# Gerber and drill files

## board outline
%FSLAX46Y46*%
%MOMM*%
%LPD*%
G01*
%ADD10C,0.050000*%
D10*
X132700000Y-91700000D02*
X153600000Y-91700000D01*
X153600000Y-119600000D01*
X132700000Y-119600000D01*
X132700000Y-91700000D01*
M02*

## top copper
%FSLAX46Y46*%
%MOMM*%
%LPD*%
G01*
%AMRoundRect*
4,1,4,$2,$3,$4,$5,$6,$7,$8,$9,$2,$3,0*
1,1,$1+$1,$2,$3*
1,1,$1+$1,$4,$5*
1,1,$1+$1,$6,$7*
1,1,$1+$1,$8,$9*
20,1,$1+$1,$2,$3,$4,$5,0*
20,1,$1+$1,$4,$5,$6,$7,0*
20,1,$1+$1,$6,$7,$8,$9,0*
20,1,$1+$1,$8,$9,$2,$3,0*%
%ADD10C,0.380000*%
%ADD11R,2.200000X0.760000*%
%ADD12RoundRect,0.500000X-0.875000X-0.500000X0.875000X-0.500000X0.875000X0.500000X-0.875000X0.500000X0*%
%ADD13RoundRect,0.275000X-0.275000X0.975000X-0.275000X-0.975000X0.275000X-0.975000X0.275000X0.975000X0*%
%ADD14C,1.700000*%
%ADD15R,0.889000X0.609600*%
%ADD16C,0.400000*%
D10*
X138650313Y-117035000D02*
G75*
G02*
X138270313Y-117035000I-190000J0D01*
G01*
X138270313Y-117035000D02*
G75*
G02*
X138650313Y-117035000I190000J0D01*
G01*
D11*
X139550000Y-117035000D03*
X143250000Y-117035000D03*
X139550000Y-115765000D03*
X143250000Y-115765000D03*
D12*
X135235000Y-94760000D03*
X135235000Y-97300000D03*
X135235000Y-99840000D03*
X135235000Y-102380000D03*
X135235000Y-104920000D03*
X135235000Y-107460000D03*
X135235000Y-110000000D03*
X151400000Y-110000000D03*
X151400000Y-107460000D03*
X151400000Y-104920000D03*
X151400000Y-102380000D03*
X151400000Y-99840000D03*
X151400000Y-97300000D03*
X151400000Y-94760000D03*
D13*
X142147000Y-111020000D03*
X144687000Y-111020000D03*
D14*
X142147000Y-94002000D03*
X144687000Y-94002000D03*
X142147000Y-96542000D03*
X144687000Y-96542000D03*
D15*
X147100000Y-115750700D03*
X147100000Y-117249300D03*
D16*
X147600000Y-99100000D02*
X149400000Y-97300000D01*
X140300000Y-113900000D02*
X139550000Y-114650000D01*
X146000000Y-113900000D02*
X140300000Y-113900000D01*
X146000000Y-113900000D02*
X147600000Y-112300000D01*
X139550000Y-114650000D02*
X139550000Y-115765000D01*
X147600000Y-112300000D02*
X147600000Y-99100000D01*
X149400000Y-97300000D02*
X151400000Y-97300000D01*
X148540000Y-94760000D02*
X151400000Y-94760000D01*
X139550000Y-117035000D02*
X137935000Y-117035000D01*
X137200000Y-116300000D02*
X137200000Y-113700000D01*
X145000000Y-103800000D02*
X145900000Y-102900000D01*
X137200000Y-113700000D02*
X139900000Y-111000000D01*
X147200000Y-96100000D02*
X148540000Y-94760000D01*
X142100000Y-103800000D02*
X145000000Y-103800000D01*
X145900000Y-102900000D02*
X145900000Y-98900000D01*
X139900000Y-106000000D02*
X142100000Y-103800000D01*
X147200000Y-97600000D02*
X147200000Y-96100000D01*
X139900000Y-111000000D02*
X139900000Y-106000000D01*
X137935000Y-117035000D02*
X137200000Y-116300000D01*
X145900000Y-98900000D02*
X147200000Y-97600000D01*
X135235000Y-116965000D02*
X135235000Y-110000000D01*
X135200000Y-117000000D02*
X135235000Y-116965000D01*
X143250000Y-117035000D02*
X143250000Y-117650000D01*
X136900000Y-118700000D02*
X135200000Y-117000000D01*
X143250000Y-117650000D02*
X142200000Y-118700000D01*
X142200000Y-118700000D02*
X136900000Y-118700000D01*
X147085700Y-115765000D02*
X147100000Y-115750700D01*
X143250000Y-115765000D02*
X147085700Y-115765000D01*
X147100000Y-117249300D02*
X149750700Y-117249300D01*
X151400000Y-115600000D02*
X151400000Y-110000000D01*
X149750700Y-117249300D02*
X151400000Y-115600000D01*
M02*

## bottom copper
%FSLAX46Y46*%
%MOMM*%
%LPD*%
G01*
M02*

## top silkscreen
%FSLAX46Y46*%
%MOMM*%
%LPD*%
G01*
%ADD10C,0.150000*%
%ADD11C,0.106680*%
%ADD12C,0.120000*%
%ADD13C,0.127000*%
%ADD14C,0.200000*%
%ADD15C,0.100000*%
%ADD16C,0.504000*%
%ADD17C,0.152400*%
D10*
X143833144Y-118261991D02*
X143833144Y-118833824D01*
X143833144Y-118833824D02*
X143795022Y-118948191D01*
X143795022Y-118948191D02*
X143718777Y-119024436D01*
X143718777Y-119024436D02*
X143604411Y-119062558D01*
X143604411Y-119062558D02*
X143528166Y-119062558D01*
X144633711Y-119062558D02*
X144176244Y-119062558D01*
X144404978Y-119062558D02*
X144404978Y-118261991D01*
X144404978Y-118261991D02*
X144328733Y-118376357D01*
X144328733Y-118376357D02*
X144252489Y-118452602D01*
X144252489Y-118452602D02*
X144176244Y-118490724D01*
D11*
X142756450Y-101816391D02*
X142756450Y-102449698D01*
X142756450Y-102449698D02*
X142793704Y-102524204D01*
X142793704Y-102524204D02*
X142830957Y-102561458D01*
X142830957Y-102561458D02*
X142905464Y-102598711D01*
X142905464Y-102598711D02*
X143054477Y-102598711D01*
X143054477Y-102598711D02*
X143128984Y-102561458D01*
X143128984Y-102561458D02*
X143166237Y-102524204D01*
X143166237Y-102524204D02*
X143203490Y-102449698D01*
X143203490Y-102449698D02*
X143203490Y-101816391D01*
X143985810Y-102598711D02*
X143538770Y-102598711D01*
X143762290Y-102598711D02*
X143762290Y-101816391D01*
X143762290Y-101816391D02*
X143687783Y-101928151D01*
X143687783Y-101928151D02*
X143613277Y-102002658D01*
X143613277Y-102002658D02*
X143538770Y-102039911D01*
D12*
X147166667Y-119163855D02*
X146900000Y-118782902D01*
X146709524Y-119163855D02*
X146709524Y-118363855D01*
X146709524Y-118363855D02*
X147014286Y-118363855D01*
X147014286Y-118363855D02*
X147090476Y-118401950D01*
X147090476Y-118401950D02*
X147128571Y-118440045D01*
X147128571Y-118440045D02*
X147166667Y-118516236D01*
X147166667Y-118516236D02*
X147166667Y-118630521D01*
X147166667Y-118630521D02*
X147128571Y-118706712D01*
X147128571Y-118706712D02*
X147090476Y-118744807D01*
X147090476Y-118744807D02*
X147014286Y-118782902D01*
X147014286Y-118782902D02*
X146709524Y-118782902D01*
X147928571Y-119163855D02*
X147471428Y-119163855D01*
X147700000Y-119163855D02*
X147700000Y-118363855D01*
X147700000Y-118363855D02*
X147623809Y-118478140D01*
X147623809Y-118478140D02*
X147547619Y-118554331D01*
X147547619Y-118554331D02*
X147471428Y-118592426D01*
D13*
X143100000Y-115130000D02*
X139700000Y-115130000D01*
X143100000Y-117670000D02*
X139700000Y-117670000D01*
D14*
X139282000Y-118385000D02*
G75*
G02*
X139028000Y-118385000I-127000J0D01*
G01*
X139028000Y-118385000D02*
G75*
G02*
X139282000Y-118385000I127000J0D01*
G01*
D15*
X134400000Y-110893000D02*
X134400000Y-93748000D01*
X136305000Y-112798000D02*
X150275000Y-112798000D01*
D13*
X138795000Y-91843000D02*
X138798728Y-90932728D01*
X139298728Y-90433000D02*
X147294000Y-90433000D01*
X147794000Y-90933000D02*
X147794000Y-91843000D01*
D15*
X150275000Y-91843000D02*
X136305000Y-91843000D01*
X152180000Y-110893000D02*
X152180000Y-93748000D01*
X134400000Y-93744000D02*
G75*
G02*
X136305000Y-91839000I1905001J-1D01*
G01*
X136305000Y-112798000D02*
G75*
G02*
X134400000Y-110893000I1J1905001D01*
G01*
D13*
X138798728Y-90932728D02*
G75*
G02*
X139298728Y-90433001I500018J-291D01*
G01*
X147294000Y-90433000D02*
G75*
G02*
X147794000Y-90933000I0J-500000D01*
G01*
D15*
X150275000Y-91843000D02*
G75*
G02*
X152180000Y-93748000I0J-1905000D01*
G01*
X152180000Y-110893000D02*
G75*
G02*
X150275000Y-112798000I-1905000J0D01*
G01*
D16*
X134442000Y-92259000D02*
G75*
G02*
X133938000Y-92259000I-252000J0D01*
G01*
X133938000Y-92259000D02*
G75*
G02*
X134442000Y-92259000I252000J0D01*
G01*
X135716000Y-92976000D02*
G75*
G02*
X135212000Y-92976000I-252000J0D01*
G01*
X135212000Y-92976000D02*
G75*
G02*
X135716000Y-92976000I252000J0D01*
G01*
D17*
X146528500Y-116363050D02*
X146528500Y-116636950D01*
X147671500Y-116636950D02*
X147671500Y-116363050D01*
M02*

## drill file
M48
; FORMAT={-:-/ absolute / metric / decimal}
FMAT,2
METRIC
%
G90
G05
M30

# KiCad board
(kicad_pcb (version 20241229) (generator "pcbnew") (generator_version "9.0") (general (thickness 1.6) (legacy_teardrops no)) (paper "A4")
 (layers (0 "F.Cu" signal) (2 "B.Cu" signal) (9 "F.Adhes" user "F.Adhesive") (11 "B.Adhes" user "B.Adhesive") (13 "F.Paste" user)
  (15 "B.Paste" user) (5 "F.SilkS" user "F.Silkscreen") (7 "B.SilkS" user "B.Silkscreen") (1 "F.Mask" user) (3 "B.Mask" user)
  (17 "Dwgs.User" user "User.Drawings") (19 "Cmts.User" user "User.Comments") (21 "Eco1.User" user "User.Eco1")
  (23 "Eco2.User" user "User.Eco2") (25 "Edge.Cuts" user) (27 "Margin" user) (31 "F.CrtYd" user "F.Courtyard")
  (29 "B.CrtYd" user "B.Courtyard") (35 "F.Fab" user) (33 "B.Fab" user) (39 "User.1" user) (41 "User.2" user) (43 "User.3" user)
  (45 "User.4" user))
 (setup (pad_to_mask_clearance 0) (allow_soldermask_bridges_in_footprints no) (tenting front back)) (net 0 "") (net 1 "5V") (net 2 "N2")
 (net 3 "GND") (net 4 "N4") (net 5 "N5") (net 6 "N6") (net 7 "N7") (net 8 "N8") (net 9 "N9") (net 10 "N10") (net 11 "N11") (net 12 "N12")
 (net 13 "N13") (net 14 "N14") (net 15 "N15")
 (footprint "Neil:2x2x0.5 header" (layer "F.Cu") (at 141.4 116.4 90)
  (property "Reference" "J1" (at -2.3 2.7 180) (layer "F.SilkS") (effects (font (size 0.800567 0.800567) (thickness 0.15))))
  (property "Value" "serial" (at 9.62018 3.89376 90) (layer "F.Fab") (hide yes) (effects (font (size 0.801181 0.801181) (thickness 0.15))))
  (fp_line (start 1.27 1.7) (end 1.27 -1.7) (stroke (width 0.127) (type solid)) (layer "F.SilkS"))
  (fp_line (start -1.27 1.7) (end -1.27 -1.7) (stroke (width 0.127) (type solid)) (layer "F.SilkS"))
  (fp_circle (center -1.985 -2.245) (end -1.858 -2.245) (stroke (width 0.2) (type solid)) (fill no) (layer "F.SilkS"))
  (pad "1" smd rect (at -0.635 -1.85 90) (size 0.76 2.2) (layers "F.Cu" "F.Mask" "F.Paste") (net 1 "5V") (solder_mask_margin 0.102))
  (pad "2" smd rect (at -0.635 1.85 90) (size 0.76 2.2) (layers "F.Cu" "F.Mask" "F.Paste") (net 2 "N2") (solder_mask_margin 0.102))
  (pad "3" smd rect (at 0.635 -1.85 90) (size 0.76 2.2) (layers "F.Cu" "F.Mask" "F.Paste") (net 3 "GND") (solder_mask_margin 0.102))
  (pad "4" smd rect (at 0.635 1.85 90) (size 0.76 2.2) (layers "F.Cu" "F.Mask" "F.Paste") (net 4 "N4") (solder_mask_margin 0.102)))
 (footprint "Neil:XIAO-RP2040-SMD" (layer "F.Cu") (at 143.235 102.38)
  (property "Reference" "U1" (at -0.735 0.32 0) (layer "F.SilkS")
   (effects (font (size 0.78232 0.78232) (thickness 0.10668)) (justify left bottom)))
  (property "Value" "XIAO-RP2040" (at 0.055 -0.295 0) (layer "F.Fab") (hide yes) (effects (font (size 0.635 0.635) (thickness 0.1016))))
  (fp_line (start -8.835 8.513) (end -8.835 -8.632) (stroke (width 0.1) (type solid)) (layer "F.SilkS"))
  (fp_line (start -6.93 10.418) (end 7.04 10.418) (stroke (width 0.1) (type solid)) (layer "F.SilkS"))
  (fp_line (start -4.44 -10.537) (end -4.436272 -11.447272) (stroke (width 0.127) (type solid)) (layer "F.SilkS"))
  (fp_line (start -3.936272 -11.947) (end 4.059 -11.947) (stroke (width 0.127) (type solid)) (layer "F.SilkS"))
  (fp_line (start 4.559 -11.447) (end 4.559 -10.537) (stroke (width 0.127) (type solid)) (layer "F.SilkS"))
  (fp_line (start 7.04 -10.537) (end -6.93 -10.537) (stroke (width 0.1) (type solid)) (layer "F.SilkS"))
  (fp_line (start 8.945 8.513) (end 8.945 -8.632) (stroke (width 0.1) (type solid)) (layer "F.SilkS"))
  (fp_arc (start -8.835 -8.636) (mid -8.277038 -9.983038) (end -6.93 -10.541) (stroke (width 0.1) (type solid)) (layer "F.SilkS"))
  (fp_arc (start -6.93 10.418) (mid -8.277038 9.860038) (end -8.835 8.513) (stroke (width 0.1) (type solid)) (layer "F.SilkS"))
  (fp_arc (start -4.436272 -11.447272) (mid -4.289724 -11.800644) (end -3.936272 -11.947) (stroke (width 0.127) (type default))
   (layer "F.SilkS"))
  (fp_arc (start 4.059 -11.947) (mid 4.412553 -11.800553) (end 4.559 -11.447) (stroke (width 0.127) (type default)) (layer "F.SilkS"))
  (fp_arc (start 7.04 -10.537) (mid 8.387038 -9.979038) (end 8.945 -8.632) (stroke (width 0.1) (type solid)) (layer "F.SilkS"))
  (fp_arc (start 8.945 8.513) (mid 8.387038 9.860038) (end 7.04 10.418) (stroke (width 0.1) (type solid)) (layer "F.SilkS"))
  (fp_circle (center -9.045 -10.121) (end -9.045 -10.375) (stroke (width 0.5) (type solid)) (fill yes) (layer "F.SilkS"))
  (fp_circle (center -7.771 -9.404) (end -7.771 -9.658) (stroke (width 0.5) (type solid)) (fill yes) (layer "F.SilkS"))
  (pad "1" smd roundrect (at -8 -7.62) (size 2.75 2) (layers "F.Cu" "F.Mask" "F.Paste") (roundrect_rratio 0.25) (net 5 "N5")
   (solder_mask_margin 0.0508) (thermal_bridge_angle 45))
  (pad "2" smd roundrect (at -8 -5.08) (size 2.75 2) (layers "F.Cu" "F.Mask" "F.Paste") (roundrect_rratio 0.25) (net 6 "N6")
   (solder_mask_margin 0.0508) (thermal_bridge_angle 45))
  (pad "3" smd roundrect (at -8 -2.54) (size 2.75 2) (layers "F.Cu" "F.Mask" "F.Paste") (roundrect_rratio 0.25) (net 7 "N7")
   (solder_mask_margin 0.0508) (thermal_bridge_angle 45))
  (pad "4" smd roundrect (at -8 0) (size 2.75 2) (layers "F.Cu" "F.Mask" "F.Paste") (roundrect_rratio 0.25) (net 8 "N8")
   (solder_mask_margin 0.0508) (thermal_bridge_angle 45))
  (pad "5" smd roundrect (at -8 2.54) (size 2.75 2) (layers "F.Cu" "F.Mask" "F.Paste") (roundrect_rratio 0.25) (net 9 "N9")
   (solder_mask_margin 0.0508) (thermal_bridge_angle 45))
  (pad "6" smd roundrect (at -8 5.08) (size 2.75 2) (layers "F.Cu" "F.Mask" "F.Paste") (roundrect_rratio 0.25) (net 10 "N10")
   (solder_mask_margin 0.0508) (thermal_bridge_angle 45))
  (pad "7" smd roundrect (at -8 7.62) (size 2.75 2) (layers "F.Cu" "F.Mask" "F.Paste") (roundrect_rratio 0.25) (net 2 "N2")
   (solder_mask_margin 0.0508) (thermal_bridge_angle 45))
  (pad "8" smd roundrect (at 8.165 7.62) (size 2.75 2) (layers "F.Cu" "F.Mask" "F.Paste") (roundrect_rratio 0.25) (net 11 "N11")
   (solder_mask_margin 0.0508) (thermal_bridge_angle 45))
  (pad "9" smd roundrect (at 8.165 5.08) (size 2.75 2) (layers "F.Cu" "F.Mask" "F.Paste") (roundrect_rratio 0.25) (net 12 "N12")
   (solder_mask_margin 0.0508) (thermal_bridge_angle 45))
  (pad "10" smd roundrect (at 8.165 2.54) (size 2.75 2) (layers "F.Cu" "F.Mask" "F.Paste") (roundrect_rratio 0.25) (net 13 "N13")
   (solder_mask_margin 0.0508) (thermal_bridge_angle 45))
  (pad "11" smd roundrect (at 8.165 0) (size 2.75 2) (layers "F.Cu" "F.Mask" "F.Paste") (roundrect_rratio 0.25) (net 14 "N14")
   (solder_mask_margin 0.0508) (thermal_bridge_angle 45))
  (pad "12" smd roundrect (at 8.165 -2.54) (size 2.75 2) (layers "F.Cu" "F.Mask" "F.Paste") (roundrect_rratio 0.25) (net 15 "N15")
   (solder_mask_margin 0.0508) (thermal_bridge_angle 45))
  (pad "13" smd roundrect (at 8.165 -5.08) (size 2.75 2) (layers "F.Cu" "F.Mask" "F.Paste") (roundrect_rratio 0.25) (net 3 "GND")
   (solder_mask_margin 0.0508) (thermal_bridge_angle 45))
  (pad "14" smd roundrect (at 8.165 -7.62) (size 2.75 2) (layers "F.Cu" "F.Mask" "F.Paste") (roundrect_rratio 0.25) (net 1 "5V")
   (solder_mask_margin 0.0508) (thermal_bridge_angle 45))
  (pad "15" smd roundrect (at -1.088 8.64 270) (size 2.5 1.1) (layers "F.Cu" "F.Mask" "F.Paste") (roundrect_rratio 0.25)
   (thermal_bridge_angle 45))
  (pad "16" smd roundrect (at 1.452 8.64 270) (size 2.5 1.1) (layers "F.Cu" "F.Mask" "F.Paste") (roundrect_rratio 0.25)
   (thermal_bridge_angle 45))
  (pad "17" smd circle (at -1.088 -8.378) (size 1.7 1.7) (layers "F.Cu" "F.Mask" "F.Paste"))
  (pad "18" smd circle (at 1.452 -8.378) (size 1.7 1.7) (layers "F.Cu" "F.Mask" "F.Paste"))
  (pad "19" smd circle (at -1.088 -5.838) (size 1.7 1.7) (layers "F.Cu" "F.Mask" "F.Paste"))
  (pad "20" smd circle (at 1.452 -5.838) (size 1.7 1.7) (layers "F.Cu" "F.Mask" "F.Paste")))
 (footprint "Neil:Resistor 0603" (layer "F.Cu") (at 147.1 116.5 -90)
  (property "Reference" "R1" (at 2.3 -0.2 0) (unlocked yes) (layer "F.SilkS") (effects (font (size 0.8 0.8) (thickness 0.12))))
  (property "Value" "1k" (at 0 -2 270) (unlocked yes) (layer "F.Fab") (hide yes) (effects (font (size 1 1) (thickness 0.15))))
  (fp_line (start -0.13695 0.5715) (end 0.13695 0.5715) (stroke (width 0.1524) (type solid)) (layer "F.SilkS"))
  (fp_line (start 0.13695 -0.5715) (end -0.13695 -0.5715) (stroke (width 0.1524) (type solid)) (layer "F.SilkS"))
  (pad "1" smd rect (at -0.7493 0 270) (size 0.6096 0.889) (layers "F.Cu" "F.Mask" "F.Paste") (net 4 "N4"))
  (pad "2" smd rect (at 0.7493 0 270) (size 0.6096 0.889) (layers "F.Cu" "F.Mask" "F.Paste") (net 11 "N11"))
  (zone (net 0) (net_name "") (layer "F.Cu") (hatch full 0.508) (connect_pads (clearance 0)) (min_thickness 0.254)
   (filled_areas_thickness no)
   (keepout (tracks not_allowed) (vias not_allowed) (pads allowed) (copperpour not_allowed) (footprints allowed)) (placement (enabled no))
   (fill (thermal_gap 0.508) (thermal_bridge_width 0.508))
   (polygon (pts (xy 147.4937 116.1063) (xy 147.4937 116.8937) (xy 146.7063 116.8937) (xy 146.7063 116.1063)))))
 (gr_circle (center 138.460313 117.035) (end 138.740313 117.035) (stroke (width 0.2) (type solid)) (fill yes) (layer "F.Cu") (net 1))
 (gr_rect (start 132.7 91.7) (end 153.6 119.6) (stroke (width 0.05) (type default)) (fill no) (layer "Edge.Cuts"))
 (segment (start 147.6 99.1) (end 149.4 97.3) (width 0.4) (layer "F.Cu") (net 3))
 (segment (start 140.3 113.9) (end 139.55 114.65) (width 0.4) (layer "F.Cu") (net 3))
 (segment (start 146 113.9) (end 140.3 113.9) (width 0.4) (layer "F.Cu") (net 3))
 (segment (start 146 113.9) (end 147.6 112.3) (width 0.4) (layer "F.Cu") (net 3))
 (segment (start 139.55 114.65) (end 139.55 115.765) (width 0.4) (layer "F.Cu") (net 3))
 (segment (start 147.6 112.3) (end 147.6 99.1) (width 0.4) (layer "F.Cu") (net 3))
 (segment (start 149.4 97.3) (end 151.4 97.3) (width 0.4) (layer "F.Cu") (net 3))
 (segment (start 148.54 94.76) (end 151.4 94.76) (width 0.4) (layer "F.Cu") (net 1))
 (segment (start 139.55 117.035) (end 137.935 117.035) (width 0.4) (layer "F.Cu") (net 1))
 (segment (start 137.2 116.3) (end 137.2 113.7) (width 0.4) (layer "F.Cu") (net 1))
 (segment (start 145 103.8) (end 145.9 102.9) (width 0.4) (layer "F.Cu") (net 1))
 (segment (start 137.2 113.7) (end 139.9 111) (width 0.4) (layer "F.Cu") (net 1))
 (segment (start 147.2 96.1) (end 148.54 94.76) (width 0.4) (layer "F.Cu") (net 1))
 (segment (start 142.1 103.8) (end 145 103.8) (width 0.4) (layer "F.Cu") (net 1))
 (segment (start 145.9 102.9) (end 145.9 98.9) (width 0.4) (layer "F.Cu") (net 1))
 (segment (start 139.9 106) (end 142.1 103.8) (width 0.4) (layer "F.Cu") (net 1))
 (segment (start 147.2 97.6) (end 147.2 96.1) (width 0.4) (layer "F.Cu") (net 1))
 (segment (start 139.9 111) (end 139.9 106) (width 0.4) (layer "F.Cu") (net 1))
 (segment (start 137.935 117.035) (end 137.2 116.3) (width 0.4) (layer "F.Cu") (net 1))
 (segment (start 145.9 98.9) (end 147.2 97.6) (width 0.4) (layer "F.Cu") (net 1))
 (segment (start 135.235 116.965) (end 135.235 110) (width 0.4) (layer "F.Cu") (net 2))
 (segment (start 135.2 117) (end 135.235 116.965) (width 0.4) (layer "F.Cu") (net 2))
 (segment (start 143.25 117.035) (end 143.25 117.65) (width 0.4) (layer "F.Cu") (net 2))
 (segment (start 136.9 118.7) (end 135.2 117) (width 0.4) (layer "F.Cu") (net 2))
 (segment (start 143.25 117.65) (end 142.2 118.7) (width 0.4) (layer "F.Cu") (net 2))
 (segment (start 142.2 118.7) (end 136.9 118.7) (width 0.4) (layer "F.Cu") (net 2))
 (segment (start 147.0857 115.765) (end 147.1 115.7507) (width 0.4) (layer "F.Cu") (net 4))
 (segment (start 143.25 115.765) (end 147.0857 115.765) (width 0.4) (layer "F.Cu") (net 4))
 (segment (start 147.1 117.2493) (end 149.7507 117.2493) (width 0.4) (layer "F.Cu") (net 11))
 (segment (start 151.4 115.6) (end 151.4 110) (width 0.4) (layer "F.Cu") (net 11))
 (segment (start 149.7507 117.2493) (end 151.4 115.6) (width 0.4) (layer "F.Cu") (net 11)))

